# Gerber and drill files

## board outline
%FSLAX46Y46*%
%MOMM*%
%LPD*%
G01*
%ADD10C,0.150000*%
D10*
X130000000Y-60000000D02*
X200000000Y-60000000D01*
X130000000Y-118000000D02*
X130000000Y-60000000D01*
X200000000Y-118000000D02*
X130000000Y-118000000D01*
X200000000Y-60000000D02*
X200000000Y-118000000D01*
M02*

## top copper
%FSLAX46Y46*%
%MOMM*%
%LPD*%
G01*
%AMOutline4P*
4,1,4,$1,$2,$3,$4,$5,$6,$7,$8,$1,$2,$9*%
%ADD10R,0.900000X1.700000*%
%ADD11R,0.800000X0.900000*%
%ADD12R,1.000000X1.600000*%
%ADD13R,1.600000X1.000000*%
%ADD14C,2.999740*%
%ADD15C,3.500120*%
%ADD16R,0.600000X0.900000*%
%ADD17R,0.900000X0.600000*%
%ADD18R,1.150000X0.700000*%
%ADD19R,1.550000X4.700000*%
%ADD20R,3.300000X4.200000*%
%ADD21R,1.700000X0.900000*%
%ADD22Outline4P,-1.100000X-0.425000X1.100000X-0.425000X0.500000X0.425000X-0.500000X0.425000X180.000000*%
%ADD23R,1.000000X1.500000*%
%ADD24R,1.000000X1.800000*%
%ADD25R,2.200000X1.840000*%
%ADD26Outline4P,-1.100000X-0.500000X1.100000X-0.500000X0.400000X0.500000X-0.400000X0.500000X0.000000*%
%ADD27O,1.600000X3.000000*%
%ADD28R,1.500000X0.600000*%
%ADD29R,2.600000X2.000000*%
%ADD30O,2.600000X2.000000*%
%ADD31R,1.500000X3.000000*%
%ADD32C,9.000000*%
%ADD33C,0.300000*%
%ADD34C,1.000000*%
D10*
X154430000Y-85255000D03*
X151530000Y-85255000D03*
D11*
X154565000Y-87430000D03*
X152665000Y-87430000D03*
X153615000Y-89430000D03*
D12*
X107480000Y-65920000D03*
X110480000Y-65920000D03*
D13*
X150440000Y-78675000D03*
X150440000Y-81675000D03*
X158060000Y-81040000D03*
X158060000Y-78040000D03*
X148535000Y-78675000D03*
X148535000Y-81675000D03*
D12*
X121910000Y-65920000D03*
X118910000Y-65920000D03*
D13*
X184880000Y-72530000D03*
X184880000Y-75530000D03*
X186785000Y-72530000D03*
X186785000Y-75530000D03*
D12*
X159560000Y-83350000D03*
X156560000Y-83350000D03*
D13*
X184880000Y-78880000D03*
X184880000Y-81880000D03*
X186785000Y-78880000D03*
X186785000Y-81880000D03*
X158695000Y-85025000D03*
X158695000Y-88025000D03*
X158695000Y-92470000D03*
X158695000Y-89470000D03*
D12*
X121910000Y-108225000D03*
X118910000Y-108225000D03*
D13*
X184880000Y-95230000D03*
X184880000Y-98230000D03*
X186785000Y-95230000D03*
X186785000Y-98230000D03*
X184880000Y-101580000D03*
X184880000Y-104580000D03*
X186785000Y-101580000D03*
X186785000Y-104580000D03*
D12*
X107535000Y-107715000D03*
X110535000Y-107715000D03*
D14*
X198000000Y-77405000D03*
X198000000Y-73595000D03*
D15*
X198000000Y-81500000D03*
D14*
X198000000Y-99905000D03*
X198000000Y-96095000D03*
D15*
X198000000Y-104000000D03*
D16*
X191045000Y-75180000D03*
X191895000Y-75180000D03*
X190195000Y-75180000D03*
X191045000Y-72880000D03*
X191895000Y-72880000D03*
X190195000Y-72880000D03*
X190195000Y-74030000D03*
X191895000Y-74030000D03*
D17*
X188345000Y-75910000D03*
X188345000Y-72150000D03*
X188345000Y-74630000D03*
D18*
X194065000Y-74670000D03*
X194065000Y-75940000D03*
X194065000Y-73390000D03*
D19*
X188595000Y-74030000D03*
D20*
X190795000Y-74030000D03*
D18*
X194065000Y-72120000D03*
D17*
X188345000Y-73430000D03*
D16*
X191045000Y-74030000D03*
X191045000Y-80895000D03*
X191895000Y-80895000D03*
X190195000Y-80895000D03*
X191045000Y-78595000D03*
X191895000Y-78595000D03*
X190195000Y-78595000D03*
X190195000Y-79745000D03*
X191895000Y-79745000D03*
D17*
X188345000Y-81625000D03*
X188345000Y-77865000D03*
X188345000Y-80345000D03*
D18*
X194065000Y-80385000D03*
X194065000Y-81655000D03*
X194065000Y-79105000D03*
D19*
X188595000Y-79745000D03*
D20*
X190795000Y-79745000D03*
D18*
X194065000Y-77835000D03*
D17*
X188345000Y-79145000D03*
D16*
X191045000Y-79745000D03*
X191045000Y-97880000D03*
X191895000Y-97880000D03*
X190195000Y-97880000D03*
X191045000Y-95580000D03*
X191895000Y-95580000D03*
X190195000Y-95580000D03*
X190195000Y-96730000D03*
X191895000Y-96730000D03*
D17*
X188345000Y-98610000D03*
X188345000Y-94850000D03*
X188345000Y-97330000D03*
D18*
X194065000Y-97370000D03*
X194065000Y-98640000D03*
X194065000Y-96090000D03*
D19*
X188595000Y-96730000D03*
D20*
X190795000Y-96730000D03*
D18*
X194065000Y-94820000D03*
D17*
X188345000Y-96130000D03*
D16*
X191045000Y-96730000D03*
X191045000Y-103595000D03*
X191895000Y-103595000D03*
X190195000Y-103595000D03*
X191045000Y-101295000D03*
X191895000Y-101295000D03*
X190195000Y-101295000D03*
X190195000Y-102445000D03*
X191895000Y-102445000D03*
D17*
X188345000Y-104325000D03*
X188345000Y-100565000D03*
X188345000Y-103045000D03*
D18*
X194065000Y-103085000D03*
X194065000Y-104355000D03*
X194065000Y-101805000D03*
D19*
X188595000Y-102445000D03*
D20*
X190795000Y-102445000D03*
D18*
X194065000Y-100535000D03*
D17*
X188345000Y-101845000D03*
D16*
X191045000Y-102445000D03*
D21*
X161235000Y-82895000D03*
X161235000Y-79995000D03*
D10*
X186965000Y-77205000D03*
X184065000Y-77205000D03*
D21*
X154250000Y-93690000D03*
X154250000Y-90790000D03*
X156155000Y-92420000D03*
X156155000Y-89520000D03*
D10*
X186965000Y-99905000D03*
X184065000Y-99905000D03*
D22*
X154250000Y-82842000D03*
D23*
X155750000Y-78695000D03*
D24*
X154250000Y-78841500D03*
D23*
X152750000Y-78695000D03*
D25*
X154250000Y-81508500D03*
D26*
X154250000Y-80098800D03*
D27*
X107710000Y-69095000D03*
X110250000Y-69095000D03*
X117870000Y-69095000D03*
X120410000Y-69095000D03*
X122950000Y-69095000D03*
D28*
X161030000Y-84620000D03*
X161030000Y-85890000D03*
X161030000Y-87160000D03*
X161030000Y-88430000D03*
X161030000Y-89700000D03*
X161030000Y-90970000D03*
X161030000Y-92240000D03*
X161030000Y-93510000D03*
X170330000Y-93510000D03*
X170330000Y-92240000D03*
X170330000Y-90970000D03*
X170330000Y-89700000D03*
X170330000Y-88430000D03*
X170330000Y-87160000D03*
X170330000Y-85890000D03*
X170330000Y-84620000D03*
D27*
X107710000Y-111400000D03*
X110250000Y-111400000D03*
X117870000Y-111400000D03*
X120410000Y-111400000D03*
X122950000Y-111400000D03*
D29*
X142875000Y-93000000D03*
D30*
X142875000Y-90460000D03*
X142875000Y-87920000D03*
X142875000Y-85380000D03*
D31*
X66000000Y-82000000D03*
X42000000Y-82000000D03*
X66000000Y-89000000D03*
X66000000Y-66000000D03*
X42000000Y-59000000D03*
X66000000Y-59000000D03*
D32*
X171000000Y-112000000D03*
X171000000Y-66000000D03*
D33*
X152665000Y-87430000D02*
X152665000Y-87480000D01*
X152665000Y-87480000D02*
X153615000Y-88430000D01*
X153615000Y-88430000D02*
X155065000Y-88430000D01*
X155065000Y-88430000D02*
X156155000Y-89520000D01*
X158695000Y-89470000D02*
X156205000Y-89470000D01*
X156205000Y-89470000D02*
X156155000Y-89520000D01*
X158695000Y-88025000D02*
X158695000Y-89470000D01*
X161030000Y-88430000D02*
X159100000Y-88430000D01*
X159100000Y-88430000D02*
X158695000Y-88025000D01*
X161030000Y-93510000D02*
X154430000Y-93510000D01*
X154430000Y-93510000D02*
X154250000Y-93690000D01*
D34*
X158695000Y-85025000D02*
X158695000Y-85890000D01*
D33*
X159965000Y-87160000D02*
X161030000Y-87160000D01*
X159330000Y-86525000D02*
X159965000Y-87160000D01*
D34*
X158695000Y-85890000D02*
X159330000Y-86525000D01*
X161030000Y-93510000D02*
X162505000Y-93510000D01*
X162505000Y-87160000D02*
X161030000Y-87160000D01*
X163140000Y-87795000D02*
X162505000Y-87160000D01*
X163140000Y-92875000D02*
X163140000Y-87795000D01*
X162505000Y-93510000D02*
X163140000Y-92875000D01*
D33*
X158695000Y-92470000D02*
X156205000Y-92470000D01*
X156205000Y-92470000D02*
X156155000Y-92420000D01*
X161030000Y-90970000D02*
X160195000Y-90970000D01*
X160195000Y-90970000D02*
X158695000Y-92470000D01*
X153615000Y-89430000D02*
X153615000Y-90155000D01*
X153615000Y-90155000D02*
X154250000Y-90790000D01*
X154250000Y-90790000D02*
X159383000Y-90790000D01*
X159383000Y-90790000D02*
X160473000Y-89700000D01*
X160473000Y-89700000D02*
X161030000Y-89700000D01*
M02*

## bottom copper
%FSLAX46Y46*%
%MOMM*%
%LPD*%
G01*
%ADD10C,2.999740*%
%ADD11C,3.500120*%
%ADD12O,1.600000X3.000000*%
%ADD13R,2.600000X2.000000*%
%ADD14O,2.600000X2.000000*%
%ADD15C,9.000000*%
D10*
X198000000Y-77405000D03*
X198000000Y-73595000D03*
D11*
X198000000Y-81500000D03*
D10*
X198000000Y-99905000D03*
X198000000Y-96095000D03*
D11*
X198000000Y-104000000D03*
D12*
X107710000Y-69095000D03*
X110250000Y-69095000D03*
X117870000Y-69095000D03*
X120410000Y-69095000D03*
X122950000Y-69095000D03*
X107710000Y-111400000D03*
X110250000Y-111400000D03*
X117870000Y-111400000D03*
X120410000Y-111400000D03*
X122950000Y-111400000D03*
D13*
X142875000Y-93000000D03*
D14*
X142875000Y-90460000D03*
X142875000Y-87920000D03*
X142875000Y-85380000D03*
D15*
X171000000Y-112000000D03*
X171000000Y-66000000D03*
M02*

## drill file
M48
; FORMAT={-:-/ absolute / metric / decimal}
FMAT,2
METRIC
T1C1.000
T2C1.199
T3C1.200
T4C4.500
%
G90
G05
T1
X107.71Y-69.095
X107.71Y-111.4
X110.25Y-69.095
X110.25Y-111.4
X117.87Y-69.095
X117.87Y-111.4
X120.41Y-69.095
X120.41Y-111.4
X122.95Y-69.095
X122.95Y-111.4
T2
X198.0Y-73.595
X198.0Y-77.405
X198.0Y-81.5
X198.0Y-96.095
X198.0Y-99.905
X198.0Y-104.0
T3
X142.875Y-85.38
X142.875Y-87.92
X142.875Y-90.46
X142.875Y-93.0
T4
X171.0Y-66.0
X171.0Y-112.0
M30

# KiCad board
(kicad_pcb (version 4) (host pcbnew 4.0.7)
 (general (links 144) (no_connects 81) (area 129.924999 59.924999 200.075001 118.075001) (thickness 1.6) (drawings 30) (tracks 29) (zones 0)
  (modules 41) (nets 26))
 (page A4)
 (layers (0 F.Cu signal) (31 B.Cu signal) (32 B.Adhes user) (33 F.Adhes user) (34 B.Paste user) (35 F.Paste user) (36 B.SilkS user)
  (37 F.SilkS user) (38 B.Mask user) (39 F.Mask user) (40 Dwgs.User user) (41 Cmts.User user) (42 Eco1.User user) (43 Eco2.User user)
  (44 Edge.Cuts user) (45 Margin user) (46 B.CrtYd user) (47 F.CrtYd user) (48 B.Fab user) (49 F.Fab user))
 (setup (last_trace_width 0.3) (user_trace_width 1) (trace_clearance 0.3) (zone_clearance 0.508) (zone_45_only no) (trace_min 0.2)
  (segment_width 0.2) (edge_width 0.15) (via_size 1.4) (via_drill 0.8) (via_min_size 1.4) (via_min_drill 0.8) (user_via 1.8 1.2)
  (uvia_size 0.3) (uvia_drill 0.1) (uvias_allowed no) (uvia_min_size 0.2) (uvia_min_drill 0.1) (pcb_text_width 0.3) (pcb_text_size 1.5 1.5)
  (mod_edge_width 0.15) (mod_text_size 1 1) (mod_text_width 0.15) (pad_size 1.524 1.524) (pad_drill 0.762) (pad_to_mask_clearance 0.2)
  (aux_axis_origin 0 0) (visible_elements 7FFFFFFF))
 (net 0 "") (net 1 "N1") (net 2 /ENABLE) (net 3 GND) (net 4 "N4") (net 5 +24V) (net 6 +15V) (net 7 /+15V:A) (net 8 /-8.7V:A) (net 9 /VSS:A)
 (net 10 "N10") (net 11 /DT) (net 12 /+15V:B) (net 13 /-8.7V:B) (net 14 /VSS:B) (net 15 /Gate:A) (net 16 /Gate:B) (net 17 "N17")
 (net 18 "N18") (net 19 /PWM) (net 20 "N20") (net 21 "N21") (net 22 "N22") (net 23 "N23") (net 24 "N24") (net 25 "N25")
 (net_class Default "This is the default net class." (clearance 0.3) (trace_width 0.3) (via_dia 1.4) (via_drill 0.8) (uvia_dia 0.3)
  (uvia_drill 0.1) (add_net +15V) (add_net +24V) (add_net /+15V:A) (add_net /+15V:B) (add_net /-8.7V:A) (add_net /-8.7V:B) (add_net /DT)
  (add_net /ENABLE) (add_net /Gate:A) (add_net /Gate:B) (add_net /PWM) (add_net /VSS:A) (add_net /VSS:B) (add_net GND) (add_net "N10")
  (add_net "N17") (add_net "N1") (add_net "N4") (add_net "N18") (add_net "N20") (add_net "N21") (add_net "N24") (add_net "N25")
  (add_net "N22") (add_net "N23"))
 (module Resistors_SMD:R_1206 (layer F.Cu) (at 152.98 85.255 180)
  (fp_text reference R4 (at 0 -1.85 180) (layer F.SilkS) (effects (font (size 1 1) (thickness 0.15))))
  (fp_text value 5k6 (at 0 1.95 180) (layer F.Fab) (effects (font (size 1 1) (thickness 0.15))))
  (pad 1 smd rect (at -1.45 0 180) (size 0.9 1.7) (layers F.Cu F.Paste F.Mask) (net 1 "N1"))
  (pad 2 smd rect (at 1.45 0 180) (size 0.9 1.7) (layers F.Cu F.Paste F.Mask) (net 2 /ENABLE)))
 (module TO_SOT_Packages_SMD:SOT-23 (layer F.Cu) (at 153.615 88.43 270)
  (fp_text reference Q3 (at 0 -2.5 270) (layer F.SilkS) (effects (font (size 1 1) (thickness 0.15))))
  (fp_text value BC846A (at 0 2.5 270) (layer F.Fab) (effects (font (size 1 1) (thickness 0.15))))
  (pad 1 smd rect (at -1 -0.95 270) (size 0.9 0.8) (layers F.Cu F.Paste F.Mask) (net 1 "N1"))
  (pad 2 smd rect (at -1 0.95 270) (size 0.9 0.8) (layers F.Cu F.Paste F.Mask) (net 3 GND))
  (pad 3 smd rect (at 1 0 270) (size 0.9 0.8) (layers F.Cu F.Paste F.Mask) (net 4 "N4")))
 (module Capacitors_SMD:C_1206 (layer F.Cu) (at 108.98 65.92)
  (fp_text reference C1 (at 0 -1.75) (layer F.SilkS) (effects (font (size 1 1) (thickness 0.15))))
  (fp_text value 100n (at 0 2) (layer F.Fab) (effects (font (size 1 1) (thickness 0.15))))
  (pad 1 smd rect (at -1.5 0) (size 1 1.6) (layers F.Cu F.Paste F.Mask) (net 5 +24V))
  (pad 2 smd rect (at 1.5 0) (size 1 1.6) (layers F.Cu F.Paste F.Mask) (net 3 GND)))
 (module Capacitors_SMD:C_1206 (layer F.Cu) (at 150.44 80.175 270)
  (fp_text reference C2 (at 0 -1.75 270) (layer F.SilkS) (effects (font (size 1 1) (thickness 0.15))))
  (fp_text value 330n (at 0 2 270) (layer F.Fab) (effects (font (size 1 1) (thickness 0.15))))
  (pad 1 smd rect (at -1.5 0 270) (size 1 1.6) (layers F.Cu F.Paste F.Mask) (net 5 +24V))
  (pad 2 smd rect (at 1.5 0 270) (size 1 1.6) (layers F.Cu F.Paste F.Mask) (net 3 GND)))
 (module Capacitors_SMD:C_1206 (layer F.Cu) (at 158.06 79.54 90)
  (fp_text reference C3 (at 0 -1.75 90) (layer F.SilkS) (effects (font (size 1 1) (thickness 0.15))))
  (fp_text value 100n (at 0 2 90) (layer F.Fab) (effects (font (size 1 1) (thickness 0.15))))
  (pad 1 smd rect (at -1.5 0 90) (size 1 1.6) (layers F.Cu F.Paste F.Mask) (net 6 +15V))
  (pad 2 smd rect (at 1.5 0 90) (size 1 1.6) (layers F.Cu F.Paste F.Mask) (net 3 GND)))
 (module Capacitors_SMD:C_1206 (layer F.Cu) (at 148.535 80.175 270)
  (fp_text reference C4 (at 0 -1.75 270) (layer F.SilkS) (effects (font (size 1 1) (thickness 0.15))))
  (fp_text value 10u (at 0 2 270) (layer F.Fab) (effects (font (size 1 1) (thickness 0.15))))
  (pad 1 smd rect (at -1.5 0 270) (size 1 1.6) (layers F.Cu F.Paste F.Mask) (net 5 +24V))
  (pad 2 smd rect (at 1.5 0 270) (size 1 1.6) (layers F.Cu F.Paste F.Mask) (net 3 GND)))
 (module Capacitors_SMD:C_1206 (layer F.Cu) (at 120.41 65.92 180)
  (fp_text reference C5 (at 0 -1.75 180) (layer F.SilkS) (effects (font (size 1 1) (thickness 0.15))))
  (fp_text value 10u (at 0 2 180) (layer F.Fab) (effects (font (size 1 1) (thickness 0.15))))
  (pad 1 smd rect (at -1.5 0 180) (size 1 1.6) (layers F.Cu F.Paste F.Mask) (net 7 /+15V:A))
  (pad 2 smd rect (at 1.5 0 180) (size 1 1.6) (layers F.Cu F.Paste F.Mask) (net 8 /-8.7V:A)))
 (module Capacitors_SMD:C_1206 (layer F.Cu) (at 184.88 74.03 270)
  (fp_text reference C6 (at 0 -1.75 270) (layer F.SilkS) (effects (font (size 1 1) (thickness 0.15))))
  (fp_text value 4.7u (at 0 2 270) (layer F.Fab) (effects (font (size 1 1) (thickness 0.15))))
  (pad 1 smd rect (at -1.5 0 270) (size 1 1.6) (layers F.Cu F.Paste F.Mask) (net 7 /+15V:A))
  (pad 2 smd rect (at 1.5 0 270) (size 1 1.6) (layers F.Cu F.Paste F.Mask) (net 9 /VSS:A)))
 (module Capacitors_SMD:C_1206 (layer F.Cu) (at 186.785 74.03 270)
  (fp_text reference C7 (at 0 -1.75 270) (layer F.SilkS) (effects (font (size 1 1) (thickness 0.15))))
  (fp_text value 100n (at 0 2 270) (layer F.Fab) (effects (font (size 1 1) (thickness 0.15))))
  (pad 1 smd rect (at -1.5 0 270) (size 1 1.6) (layers F.Cu F.Paste F.Mask) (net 7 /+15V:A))
  (pad 2 smd rect (at 1.5 0 270) (size 1 1.6) (layers F.Cu F.Paste F.Mask) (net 9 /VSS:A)))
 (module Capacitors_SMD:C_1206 (layer F.Cu) (at 158.06 83.35 180)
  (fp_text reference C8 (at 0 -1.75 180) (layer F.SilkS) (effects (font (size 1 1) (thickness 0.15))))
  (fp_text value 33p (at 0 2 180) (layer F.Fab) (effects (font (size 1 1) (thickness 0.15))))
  (pad 1 smd rect (at -1.5 0 180) (size 1 1.6) (layers F.Cu F.Paste F.Mask) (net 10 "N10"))
  (pad 2 smd rect (at 1.5 0 180) (size 1 1.6) (layers F.Cu F.Paste F.Mask) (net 3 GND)))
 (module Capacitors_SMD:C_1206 (layer F.Cu) (at 184.88 80.38 270)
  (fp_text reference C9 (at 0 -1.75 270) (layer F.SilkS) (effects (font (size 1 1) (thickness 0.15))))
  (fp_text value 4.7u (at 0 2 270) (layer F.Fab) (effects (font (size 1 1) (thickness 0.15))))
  (pad 1 smd rect (at -1.5 0 270) (size 1 1.6) (layers F.Cu F.Paste F.Mask) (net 9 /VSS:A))
  (pad 2 smd rect (at 1.5 0 270) (size 1 1.6) (layers F.Cu F.Paste F.Mask) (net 8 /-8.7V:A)))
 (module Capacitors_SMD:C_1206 (layer F.Cu) (at 186.785 80.38 270)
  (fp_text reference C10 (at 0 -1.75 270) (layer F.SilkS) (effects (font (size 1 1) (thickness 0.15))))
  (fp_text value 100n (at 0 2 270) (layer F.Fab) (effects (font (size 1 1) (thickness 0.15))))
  (pad 1 smd rect (at -1.5 0 270) (size 1 1.6) (layers F.Cu F.Paste F.Mask) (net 9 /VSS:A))
  (pad 2 smd rect (at 1.5 0 270) (size 1 1.6) (layers F.Cu F.Paste F.Mask) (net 8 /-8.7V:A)))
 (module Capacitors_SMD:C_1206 (layer F.Cu) (at 158.695 86.525 270)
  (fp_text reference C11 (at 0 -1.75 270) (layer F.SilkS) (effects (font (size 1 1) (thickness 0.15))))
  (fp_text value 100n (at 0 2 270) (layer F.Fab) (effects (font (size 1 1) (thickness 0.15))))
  (pad 1 smd rect (at -1.5 0 270) (size 1 1.6) (layers F.Cu F.Paste F.Mask) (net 6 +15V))
  (pad 2 smd rect (at 1.5 0 270) (size 1 1.6) (layers F.Cu F.Paste F.Mask) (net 3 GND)))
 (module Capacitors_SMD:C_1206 (layer F.Cu) (at 158.695 90.97 90)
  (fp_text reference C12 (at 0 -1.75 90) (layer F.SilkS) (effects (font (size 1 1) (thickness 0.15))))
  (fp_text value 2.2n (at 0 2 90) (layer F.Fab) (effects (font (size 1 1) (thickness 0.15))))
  (pad 1 smd rect (at -1.5 0 90) (size 1 1.6) (layers F.Cu F.Paste F.Mask) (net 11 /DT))
  (pad 2 smd rect (at 1.5 0 90) (size 1 1.6) (layers F.Cu F.Paste F.Mask) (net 3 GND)))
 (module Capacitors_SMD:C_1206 (layer F.Cu) (at 120.41 108.225 180)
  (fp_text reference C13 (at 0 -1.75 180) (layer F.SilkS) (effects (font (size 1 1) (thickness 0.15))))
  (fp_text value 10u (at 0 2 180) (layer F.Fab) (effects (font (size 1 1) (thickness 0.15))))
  (pad 1 smd rect (at -1.5 0 180) (size 1 1.6) (layers F.Cu F.Paste F.Mask) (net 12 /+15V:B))
  (pad 2 smd rect (at 1.5 0 180) (size 1 1.6) (layers F.Cu F.Paste F.Mask) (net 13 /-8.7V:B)))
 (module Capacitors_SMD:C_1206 (layer F.Cu) (at 184.88 96.73 270)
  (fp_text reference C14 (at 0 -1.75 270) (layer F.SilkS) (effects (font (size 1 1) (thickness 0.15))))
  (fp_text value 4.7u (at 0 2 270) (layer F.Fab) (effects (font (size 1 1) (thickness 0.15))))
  (pad 1 smd rect (at -1.5 0 270) (size 1 1.6) (layers F.Cu F.Paste F.Mask) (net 12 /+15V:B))
  (pad 2 smd rect (at 1.5 0 270) (size 1 1.6) (layers F.Cu F.Paste F.Mask) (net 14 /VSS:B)))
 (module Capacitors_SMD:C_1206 (layer F.Cu) (at 186.785 96.73 270)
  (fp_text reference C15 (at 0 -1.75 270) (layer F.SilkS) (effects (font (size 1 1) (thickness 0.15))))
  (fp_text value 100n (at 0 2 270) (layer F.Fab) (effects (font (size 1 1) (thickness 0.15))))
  (pad 1 smd rect (at -1.5 0 270) (size 1 1.6) (layers F.Cu F.Paste F.Mask) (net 12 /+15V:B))
  (pad 2 smd rect (at 1.5 0 270) (size 1 1.6) (layers F.Cu F.Paste F.Mask) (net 14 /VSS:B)))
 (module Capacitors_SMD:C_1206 (layer F.Cu) (at 184.88 103.08 270)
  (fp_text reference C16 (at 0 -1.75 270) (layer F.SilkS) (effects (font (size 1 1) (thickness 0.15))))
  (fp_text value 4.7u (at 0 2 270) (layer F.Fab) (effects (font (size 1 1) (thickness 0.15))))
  (pad 1 smd rect (at -1.5 0 270) (size 1 1.6) (layers F.Cu F.Paste F.Mask) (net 14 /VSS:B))
  (pad 2 smd rect (at 1.5 0 270) (size 1 1.6) (layers F.Cu F.Paste F.Mask) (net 13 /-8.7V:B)))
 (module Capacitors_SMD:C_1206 (layer F.Cu) (at 186.785 103.08 270)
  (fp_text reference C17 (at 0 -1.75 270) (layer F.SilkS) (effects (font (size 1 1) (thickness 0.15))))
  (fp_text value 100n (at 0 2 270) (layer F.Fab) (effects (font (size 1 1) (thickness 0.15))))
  (pad 1 smd rect (at -1.5 0 270) (size 1 1.6) (layers F.Cu F.Paste F.Mask) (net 14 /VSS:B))
  (pad 2 smd rect (at 1.5 0 270) (size 1 1.6) (layers F.Cu F.Paste F.Mask) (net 13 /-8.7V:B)))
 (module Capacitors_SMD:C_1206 (layer F.Cu) (at 109.035 107.715)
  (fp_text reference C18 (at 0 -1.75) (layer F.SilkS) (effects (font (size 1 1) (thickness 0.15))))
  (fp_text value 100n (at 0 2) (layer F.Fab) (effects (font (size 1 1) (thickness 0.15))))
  (pad 1 smd rect (at -1.5 0) (size 1 1.6) (layers F.Cu F.Paste F.Mask) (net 5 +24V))
  (pad 2 smd rect (at 1.5 0) (size 1 1.6) (layers F.Cu F.Paste F.Mask) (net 3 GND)))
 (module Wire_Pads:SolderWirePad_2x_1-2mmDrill (layer F.Cu) (at 198 75.5 90)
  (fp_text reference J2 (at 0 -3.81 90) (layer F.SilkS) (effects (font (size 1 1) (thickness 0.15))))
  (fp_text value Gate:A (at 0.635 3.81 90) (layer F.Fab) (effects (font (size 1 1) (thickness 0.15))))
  (pad 1 thru_hole circle (at -1.905 0 90) (size 2.99974 2.99974) (drill 1.19888) (layers *.Cu *.Mask) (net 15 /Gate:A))
  (pad 1 thru_hole circle (at 1.905 0 90) (size 2.99974 2.99974) (drill 1.19888) (layers *.Cu *.Mask) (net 15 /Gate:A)))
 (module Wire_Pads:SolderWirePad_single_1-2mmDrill (layer F.Cu) (at 198 81.5)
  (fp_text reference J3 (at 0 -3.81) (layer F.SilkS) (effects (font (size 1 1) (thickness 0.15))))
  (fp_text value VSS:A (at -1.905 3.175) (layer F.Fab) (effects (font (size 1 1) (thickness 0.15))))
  (pad 1 thru_hole circle (at 0 0) (size 3.50012 3.50012) (drill 1.19888) (layers *.Cu *.Mask) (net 9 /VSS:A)))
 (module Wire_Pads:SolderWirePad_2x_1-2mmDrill (layer F.Cu) (at 198 98 90)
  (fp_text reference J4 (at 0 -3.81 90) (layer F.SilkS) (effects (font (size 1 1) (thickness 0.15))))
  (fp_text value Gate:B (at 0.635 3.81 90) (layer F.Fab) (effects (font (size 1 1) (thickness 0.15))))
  (pad 1 thru_hole circle (at -1.905 0 90) (size 2.99974 2.99974) (drill 1.19888) (layers *.Cu *.Mask) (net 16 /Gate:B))
  (pad 1 thru_hole circle (at 1.905 0 90) (size 2.99974 2.99974) (drill 1.19888) (layers *.Cu *.Mask) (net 16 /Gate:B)))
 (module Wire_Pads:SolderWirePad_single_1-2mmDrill (layer F.Cu) (at 198 104)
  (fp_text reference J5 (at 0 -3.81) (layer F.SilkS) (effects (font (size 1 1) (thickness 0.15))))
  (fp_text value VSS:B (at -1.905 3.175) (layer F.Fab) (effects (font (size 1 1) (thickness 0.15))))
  (pad 1 thru_hole circle (at 0 0) (size 3.50012 3.50012) (drill 1.19888) (layers *.Cu *.Mask) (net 14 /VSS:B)))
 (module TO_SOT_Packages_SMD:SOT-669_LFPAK (layer F.Cu) (at 191.23 74.03 180) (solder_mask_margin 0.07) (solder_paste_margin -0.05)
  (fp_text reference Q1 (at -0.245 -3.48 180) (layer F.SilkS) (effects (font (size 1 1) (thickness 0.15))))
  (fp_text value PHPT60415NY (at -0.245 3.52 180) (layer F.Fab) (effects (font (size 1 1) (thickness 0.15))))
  (pad 5 smd rect (at 0.185 -1.15 180) (size 0.6 0.9) (layers F.Cu F.Paste F.Mask) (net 7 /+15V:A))
  (pad 5 smd rect (at -0.665 -1.15 180) (size 0.6 0.9) (layers F.Cu F.Paste F.Mask) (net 7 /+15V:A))
  (pad 5 smd rect (at 1.035 -1.15 180) (size 0.6 0.9) (layers F.Cu F.Paste F.Mask) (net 7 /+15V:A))
  (pad 5 smd rect (at 0.185 1.15 180) (size 0.6 0.9) (layers F.Cu F.Paste F.Mask) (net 7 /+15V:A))
  (pad 5 smd rect (at -0.665 1.15 180) (size 0.6 0.9) (layers F.Cu F.Paste F.Mask) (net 7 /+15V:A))
  (pad 5 smd rect (at 1.035 1.15 180) (size 0.6 0.9) (layers F.Cu F.Paste F.Mask) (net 7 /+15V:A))
  (pad 5 smd rect (at 1.035 0 180) (size 0.6 0.9) (layers F.Cu F.Paste F.Mask) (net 7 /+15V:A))
  (pad 5 smd rect (at -0.665 0 180) (size 0.6 0.9) (layers F.Cu F.Paste F.Mask) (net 7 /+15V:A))
  (pad 5 smd rect (at 2.885 -1.88 90) (size 0.6 0.9) (layers F.Cu F.Paste F.Mask) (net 7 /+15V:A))
  (pad 5 smd rect (at 2.885 1.88 90) (size 0.6 0.9) (layers F.Cu F.Paste F.Mask) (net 7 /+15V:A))
  (pad 5 smd rect (at 2.885 -0.6 90) (size 0.6 0.9) (layers F.Cu F.Paste F.Mask) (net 7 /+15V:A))
  (pad 2 smd rect (at -2.835 -0.64 90) (size 0.7 1.15) (layers F.Cu F.Paste F.Mask) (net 15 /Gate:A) (solder_mask_margin 0.07)
   (solder_paste_margin -0.05))
  (pad 1 smd rect (at -2.835 -1.91 90) (size 0.7 1.15) (layers F.Cu F.Paste F.Mask) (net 15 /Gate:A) (solder_mask_margin 0.07)
   (solder_paste_margin -0.05))
  (pad 3 smd rect (at -2.835 0.64 90) (size 0.7 1.15) (layers F.Cu F.Paste F.Mask) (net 15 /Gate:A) (solder_mask_margin 0.07)
   (solder_paste_margin -0.05))
  (pad 5 smd rect (at 2.635 0 90) (size 4.7 1.55) (layers F.Cu F.Paste F.Mask) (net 7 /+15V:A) (solder_mask_margin 0.07))
  (pad 5 smd rect (at 0.435 0 90) (size 4.2 3.3) (layers F.Cu F.Paste F.Mask) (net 7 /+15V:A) (solder_mask_margin 0.07))
  (pad 4 smd rect (at -2.835 1.91 90) (size 0.7 1.15) (layers F.Cu F.Paste F.Mask) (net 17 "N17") (solder_mask_margin 0.07)
   (solder_paste_margin -0.05))
  (pad 5 smd rect (at 2.885 0.6 90) (size 0.6 0.9) (layers F.Cu F.Paste F.Mask) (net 7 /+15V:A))
  (pad 5 smd rect (at 0.185 0 180) (size 0.6 0.9) (layers F.Cu F.Paste F.Mask) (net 7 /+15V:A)))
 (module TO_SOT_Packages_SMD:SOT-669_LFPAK (layer F.Cu) (at 191.23 79.745 180) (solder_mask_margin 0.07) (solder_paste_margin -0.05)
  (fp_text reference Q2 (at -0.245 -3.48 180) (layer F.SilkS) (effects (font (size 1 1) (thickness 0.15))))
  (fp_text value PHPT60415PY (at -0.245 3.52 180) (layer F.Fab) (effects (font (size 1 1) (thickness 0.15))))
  (pad 5 smd rect (at 0.185 -1.15 180) (size 0.6 0.9) (layers F.Cu F.Paste F.Mask) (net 8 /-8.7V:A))
  (pad 5 smd rect (at -0.665 -1.15 180) (size 0.6 0.9) (layers F.Cu F.Paste F.Mask) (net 8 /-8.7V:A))
  (pad 5 smd rect (at 1.035 -1.15 180) (size 0.6 0.9) (layers F.Cu F.Paste F.Mask) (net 8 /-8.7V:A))
  (pad 5 smd rect (at 0.185 1.15 180) (size 0.6 0.9) (layers F.Cu F.Paste F.Mask) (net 8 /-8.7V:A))
  (pad 5 smd rect (at -0.665 1.15 180) (size 0.6 0.9) (layers F.Cu F.Paste F.Mask) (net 8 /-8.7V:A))
  (pad 5 smd rect (at 1.035 1.15 180) (size 0.6 0.9) (layers F.Cu F.Paste F.Mask) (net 8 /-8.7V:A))
  (pad 5 smd rect (at 1.035 0 180) (size 0.6 0.9) (layers F.Cu F.Paste F.Mask) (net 8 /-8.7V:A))
  (pad 5 smd rect (at -0.665 0 180) (size 0.6 0.9) (layers F.Cu F.Paste F.Mask) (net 8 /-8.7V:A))
  (pad 5 smd rect (at 2.885 -1.88 90) (size 0.6 0.9) (layers F.Cu F.Paste F.Mask) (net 8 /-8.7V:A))
  (pad 5 smd rect (at 2.885 1.88 90) (size 0.6 0.9) (layers F.Cu F.Paste F.Mask) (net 8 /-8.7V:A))
  (pad 5 smd rect (at 2.885 -0.6 90) (size 0.6 0.9) (layers F.Cu F.Paste F.Mask) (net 8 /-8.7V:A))
  (pad 2 smd rect (at -2.835 -0.64 90) (size 0.7 1.15) (layers F.Cu F.Paste F.Mask) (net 15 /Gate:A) (solder_mask_margin 0.07)
   (solder_paste_margin -0.05))
  (pad 1 smd rect (at -2.835 -1.91 90) (size 0.7 1.15) (layers F.Cu F.Paste F.Mask) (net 15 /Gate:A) (solder_mask_margin 0.07)
   (solder_paste_margin -0.05))
  (pad 3 smd rect (at -2.835 0.64 90) (size 0.7 1.15) (layers F.Cu F.Paste F.Mask) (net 15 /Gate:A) (solder_mask_margin 0.07)
   (solder_paste_margin -0.05))
  (pad 5 smd rect (at 2.635 0 90) (size 4.7 1.55) (layers F.Cu F.Paste F.Mask) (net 8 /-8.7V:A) (solder_mask_margin 0.07))
  (pad 5 smd rect (at 0.435 0 90) (size 4.2 3.3) (layers F.Cu F.Paste F.Mask) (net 8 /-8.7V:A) (solder_mask_margin 0.07))
  (pad 4 smd rect (at -2.835 1.91 90) (size 0.7 1.15) (layers F.Cu F.Paste F.Mask) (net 17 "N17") (solder_mask_margin 0.07)
   (solder_paste_margin -0.05))
  (pad 5 smd rect (at 2.885 0.6 90) (size 0.6 0.9) (layers F.Cu F.Paste F.Mask) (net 8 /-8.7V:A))
  (pad 5 smd rect (at 0.185 0 180) (size 0.6 0.9) (layers F.Cu F.Paste F.Mask) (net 8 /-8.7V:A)))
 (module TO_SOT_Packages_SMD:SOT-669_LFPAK (layer F.Cu) (at 191.23 96.73 180) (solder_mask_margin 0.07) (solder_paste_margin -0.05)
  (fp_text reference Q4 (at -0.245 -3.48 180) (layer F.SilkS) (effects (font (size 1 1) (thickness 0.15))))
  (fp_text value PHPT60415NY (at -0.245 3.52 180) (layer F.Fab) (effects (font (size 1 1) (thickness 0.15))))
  (pad 5 smd rect (at 0.185 -1.15 180) (size 0.6 0.9) (layers F.Cu F.Paste F.Mask) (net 12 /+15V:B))
  (pad 5 smd rect (at -0.665 -1.15 180) (size 0.6 0.9) (layers F.Cu F.Paste F.Mask) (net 12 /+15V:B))
  (pad 5 smd rect (at 1.035 -1.15 180) (size 0.6 0.9) (layers F.Cu F.Paste F.Mask) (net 12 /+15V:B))
  (pad 5 smd rect (at 0.185 1.15 180) (size 0.6 0.9) (layers F.Cu F.Paste F.Mask) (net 12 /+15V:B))
  (pad 5 smd rect (at -0.665 1.15 180) (size 0.6 0.9) (layers F.Cu F.Paste F.Mask) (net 12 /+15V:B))
  (pad 5 smd rect (at 1.035 1.15 180) (size 0.6 0.9) (layers F.Cu F.Paste F.Mask) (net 12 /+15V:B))
  (pad 5 smd rect (at 1.035 0 180) (size 0.6 0.9) (layers F.Cu F.Paste F.Mask) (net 12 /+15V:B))
  (pad 5 smd rect (at -0.665 0 180) (size 0.6 0.9) (layers F.Cu F.Paste F.Mask) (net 12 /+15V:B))
  (pad 5 smd rect (at 2.885 -1.88 90) (size 0.6 0.9) (layers F.Cu F.Paste F.Mask) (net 12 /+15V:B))
  (pad 5 smd rect (at 2.885 1.88 90) (size 0.6 0.9) (layers F.Cu F.Paste F.Mask) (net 12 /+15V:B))
  (pad 5 smd rect (at 2.885 -0.6 90) (size 0.6 0.9) (layers F.Cu F.Paste F.Mask) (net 12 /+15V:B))
  (pad 2 smd rect (at -2.835 -0.64 90) (size 0.7 1.15) (layers F.Cu F.Paste F.Mask) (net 16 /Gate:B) (solder_mask_margin 0.07)
   (solder_paste_margin -0.05))
  (pad 1 smd rect (at -2.835 -1.91 90) (size 0.7 1.15) (layers F.Cu F.Paste F.Mask) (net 16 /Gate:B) (solder_mask_margin 0.07)
   (solder_paste_margin -0.05))
  (pad 3 smd rect (at -2.835 0.64 90) (size 0.7 1.15) (layers F.Cu F.Paste F.Mask) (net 16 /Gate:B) (solder_mask_margin 0.07)
   (solder_paste_margin -0.05))
  (pad 5 smd rect (at 2.635 0 90) (size 4.7 1.55) (layers F.Cu F.Paste F.Mask) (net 12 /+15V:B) (solder_mask_margin 0.07))
  (pad 5 smd rect (at 0.435 0 90) (size 4.2 3.3) (layers F.Cu F.Paste F.Mask) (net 12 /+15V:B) (solder_mask_margin 0.07))
  (pad 4 smd rect (at -2.835 1.91 90) (size 0.7 1.15) (layers F.Cu F.Paste F.Mask) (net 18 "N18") (solder_mask_margin 0.07)
   (solder_paste_margin -0.05))
  (pad 5 smd rect (at 2.885 0.6 90) (size 0.6 0.9) (layers F.Cu F.Paste F.Mask) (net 12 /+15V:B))
  (pad 5 smd rect (at 0.185 0 180) (size 0.6 0.9) (layers F.Cu F.Paste F.Mask) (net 12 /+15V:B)))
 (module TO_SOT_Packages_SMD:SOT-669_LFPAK (layer F.Cu) (at 191.23 102.445 180) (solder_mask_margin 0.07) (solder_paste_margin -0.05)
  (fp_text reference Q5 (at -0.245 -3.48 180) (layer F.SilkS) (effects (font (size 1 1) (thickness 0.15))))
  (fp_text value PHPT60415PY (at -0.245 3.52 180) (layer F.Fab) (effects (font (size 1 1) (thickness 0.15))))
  (pad 5 smd rect (at 0.185 -1.15 180) (size 0.6 0.9) (layers F.Cu F.Paste F.Mask) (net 13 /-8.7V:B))
  (pad 5 smd rect (at -0.665 -1.15 180) (size 0.6 0.9) (layers F.Cu F.Paste F.Mask) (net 13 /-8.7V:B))
  (pad 5 smd rect (at 1.035 -1.15 180) (size 0.6 0.9) (layers F.Cu F.Paste F.Mask) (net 13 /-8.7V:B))
  (pad 5 smd rect (at 0.185 1.15 180) (size 0.6 0.9) (layers F.Cu F.Paste F.Mask) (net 13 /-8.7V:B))
  (pad 5 smd rect (at -0.665 1.15 180) (size 0.6 0.9) (layers F.Cu F.Paste F.Mask) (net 13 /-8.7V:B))
  (pad 5 smd rect (at 1.035 1.15 180) (size 0.6 0.9) (layers F.Cu F.Paste F.Mask) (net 13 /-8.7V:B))
  (pad 5 smd rect (at 1.035 0 180) (size 0.6 0.9) (layers F.Cu F.Paste F.Mask) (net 13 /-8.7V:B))
  (pad 5 smd rect (at -0.665 0 180) (size 0.6 0.9) (layers F.Cu F.Paste F.Mask) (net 13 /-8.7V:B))
  (pad 5 smd rect (at 2.885 -1.88 90) (size 0.6 0.9) (layers F.Cu F.Paste F.Mask) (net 13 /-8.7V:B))
  (pad 5 smd rect (at 2.885 1.88 90) (size 0.6 0.9) (layers F.Cu F.Paste F.Mask) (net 13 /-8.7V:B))
  (pad 5 smd rect (at 2.885 -0.6 90) (size 0.6 0.9) (layers F.Cu F.Paste F.Mask) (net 13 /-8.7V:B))
  (pad 2 smd rect (at -2.835 -0.64 90) (size 0.7 1.15) (layers F.Cu F.Paste F.Mask) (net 16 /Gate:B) (solder_mask_margin 0.07)
   (solder_paste_margin -0.05))
  (pad 1 smd rect (at -2.835 -1.91 90) (size 0.7 1.15) (layers F.Cu F.Paste F.Mask) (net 16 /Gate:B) (solder_mask_margin 0.07)
   (solder_paste_margin -0.05))
  (pad 3 smd rect (at -2.835 0.64 90) (size 0.7 1.15) (layers F.Cu F.Paste F.Mask) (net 16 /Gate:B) (solder_mask_margin 0.07)
   (solder_paste_margin -0.05))
  (pad 5 smd rect (at 2.635 0 90) (size 4.7 1.55) (layers F.Cu F.Paste F.Mask) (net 13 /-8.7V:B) (solder_mask_margin 0.07))
  (pad 5 smd rect (at 0.435 0 90) (size 4.2 3.3) (layers F.Cu F.Paste F.Mask) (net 13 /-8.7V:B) (solder_mask_margin 0.07))
  (pad 4 smd rect (at -2.835 1.91 90) (size 0.7 1.15) (layers F.Cu F.Paste F.Mask) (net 18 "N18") (solder_mask_margin 0.07)
   (solder_paste_margin -0.05))
  (pad 5 smd rect (at 2.885 0.6 90) (size 0.6 0.9) (layers F.Cu F.Paste F.Mask) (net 13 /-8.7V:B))
  (pad 5 smd rect (at 0.185 0 180) (size 0.6 0.9) (layers F.Cu F.Paste F.Mask) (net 13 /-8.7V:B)))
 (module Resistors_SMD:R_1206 (layer F.Cu) (at 161.235 81.445 90)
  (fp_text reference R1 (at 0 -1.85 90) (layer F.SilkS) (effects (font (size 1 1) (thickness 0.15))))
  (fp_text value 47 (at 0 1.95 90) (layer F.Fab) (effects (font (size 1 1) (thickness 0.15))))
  (pad 1 smd rect (at -1.45 0 90) (size 0.9 1.7) (layers F.Cu F.Paste F.Mask) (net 10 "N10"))
  (pad 2 smd rect (at 1.45 0 90) (size 0.9 1.7) (layers F.Cu F.Paste F.Mask) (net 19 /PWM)))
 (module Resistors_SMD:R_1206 (layer F.Cu) (at 185.515 77.205 180)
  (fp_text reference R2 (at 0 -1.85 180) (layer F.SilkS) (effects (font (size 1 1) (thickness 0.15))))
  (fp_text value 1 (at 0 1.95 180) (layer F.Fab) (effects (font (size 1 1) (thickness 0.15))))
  (pad 1 smd rect (at -1.45 0 180) (size 0.9 1.7) (layers F.Cu F.Paste F.Mask) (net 17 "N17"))
  (pad 2 smd rect (at 1.45 0 180) (size 0.9 1.7) (layers F.Cu F.Paste F.Mask) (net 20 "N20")))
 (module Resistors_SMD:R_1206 (layer F.Cu) (at 154.25 92.24 90)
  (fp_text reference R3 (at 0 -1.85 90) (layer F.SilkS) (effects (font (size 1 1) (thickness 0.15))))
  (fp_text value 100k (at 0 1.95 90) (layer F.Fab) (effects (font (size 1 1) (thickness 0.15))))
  (pad 1 smd rect (at -1.45 0 90) (size 0.9 1.7) (layers F.Cu F.Paste F.Mask) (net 6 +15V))
  (pad 2 smd rect (at 1.45 0 90) (size 0.9 1.7) (layers F.Cu F.Paste F.Mask) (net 4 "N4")))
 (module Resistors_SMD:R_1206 (layer F.Cu) (at 156.155 90.97 90)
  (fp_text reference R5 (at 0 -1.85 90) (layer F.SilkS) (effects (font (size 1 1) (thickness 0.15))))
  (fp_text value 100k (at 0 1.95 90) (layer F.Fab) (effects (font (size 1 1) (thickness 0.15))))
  (pad 1 smd rect (at -1.45 0 90) (size 0.9 1.7) (layers F.Cu F.Paste F.Mask) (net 11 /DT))
  (pad 2 smd rect (at 1.45 0 90) (size 0.9 1.7) (layers F.Cu F.Paste F.Mask) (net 3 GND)))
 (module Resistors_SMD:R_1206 (layer F.Cu) (at 185.515 99.905 180)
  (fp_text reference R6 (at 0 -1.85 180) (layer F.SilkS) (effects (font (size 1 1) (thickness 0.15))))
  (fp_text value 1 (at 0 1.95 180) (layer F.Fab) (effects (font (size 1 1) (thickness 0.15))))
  (pad 1 smd rect (at -1.45 0 180) (size 0.9 1.7) (layers F.Cu F.Paste F.Mask) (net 18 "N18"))
  (pad 2 smd rect (at 1.45 0 180) (size 0.9 1.7) (layers F.Cu F.Paste F.Mask) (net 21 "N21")))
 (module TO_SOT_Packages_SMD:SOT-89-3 (layer F.Cu) (at 154.25 80.175 270)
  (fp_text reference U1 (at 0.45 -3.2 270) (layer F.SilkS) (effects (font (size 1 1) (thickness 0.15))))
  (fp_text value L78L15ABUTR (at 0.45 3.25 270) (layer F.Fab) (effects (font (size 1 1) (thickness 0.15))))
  (pad 2 smd trapezoid (at 2.667 0 180) (size 1.6 0.85) (rect_delta 0 0.6) (layers F.Cu F.Paste F.Mask) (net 3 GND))
  (pad 1 smd rect (at -1.48 -1.5 180) (size 1 1.5) (layers F.Cu F.Paste F.Mask) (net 6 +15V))
  (pad 2 smd rect (at -1.3335 0 180) (size 1 1.8) (layers F.Cu F.Paste F.Mask) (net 3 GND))
  (pad 3 smd rect (at -1.48 1.5 180) (size 1 1.5) (layers F.Cu F.Paste F.Mask) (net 5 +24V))
  (pad 2 smd rect (at 1.3335 0 180) (size 2.2 1.84) (layers F.Cu F.Paste F.Mask) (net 3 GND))
  (pad 2 smd trapezoid (at -0.0762 0) (size 1.5 1) (rect_delta 0 0.7) (layers F.Cu F.Paste F.Mask) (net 3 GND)))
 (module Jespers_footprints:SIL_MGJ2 (layer B.Cu) (at 107.71 69.095)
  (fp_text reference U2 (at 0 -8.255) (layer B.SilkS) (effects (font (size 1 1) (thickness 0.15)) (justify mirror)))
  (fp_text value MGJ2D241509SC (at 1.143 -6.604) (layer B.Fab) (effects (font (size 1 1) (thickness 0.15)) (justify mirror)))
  (pad 1 thru_hole oval (at 0 0) (size 1.6 3) (drill 1) (layers *.Cu *.Mask) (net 5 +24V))
  (pad 2 thru_hole oval (at 2.54 0) (size 1.6 3) (drill 1) (layers *.Cu *.Mask) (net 3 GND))
  (pad 5 thru_hole oval (at 10.16 0) (size 1.6 3) (drill 1) (layers *.Cu *.Mask) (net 8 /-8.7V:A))
  (pad 6 thru_hole oval (at 12.7 0) (size 1.6 3) (drill 1) (layers *.Cu *.Mask) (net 9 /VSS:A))
  (pad 7 thru_hole oval (at 15.24 0) (size 1.6 3) (drill 1) (layers *.Cu *.Mask) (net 7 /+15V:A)))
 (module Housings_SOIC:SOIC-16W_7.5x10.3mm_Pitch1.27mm (layer F.Cu) (at 165.68 89.065)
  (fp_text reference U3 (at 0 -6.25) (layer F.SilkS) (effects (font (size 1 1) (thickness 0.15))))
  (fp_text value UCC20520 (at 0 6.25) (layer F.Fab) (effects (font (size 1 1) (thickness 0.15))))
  (pad 1 smd rect (at -4.65 -4.445) (size 1.5 0.6) (layers F.Cu F.Paste F.Mask) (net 10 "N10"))
  (pad 2 smd rect (at -4.65 -3.175) (size 1.5 0.6) (layers F.Cu F.Paste F.Mask) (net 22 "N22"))
  (pad 3 smd rect (at -4.65 -1.905) (size 1.5 0.6) (layers F.Cu F.Paste F.Mask) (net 6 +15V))
  (pad 4 smd rect (at -4.65 -0.635) (size 1.5 0.6) (layers F.Cu F.Paste F.Mask) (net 3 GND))
  (pad 5 smd rect (at -4.65 0.635) (size 1.5 0.6) (layers F.Cu F.Paste F.Mask) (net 4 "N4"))
  (pad 6 smd rect (at -4.65 1.905) (size 1.5 0.6) (layers F.Cu F.Paste F.Mask) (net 11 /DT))
  (pad 7 smd rect (at -4.65 3.175) (size 1.5 0.6) (layers F.Cu F.Paste F.Mask) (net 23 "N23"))
  (pad 8 smd rect (at -4.65 4.445) (size 1.5 0.6) (layers F.Cu F.Paste F.Mask) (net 6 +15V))
  (pad 9 smd rect (at 4.65 4.445) (size 1.5 0.6) (layers F.Cu F.Paste F.Mask) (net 13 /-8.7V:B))
  (pad 10 smd rect (at 4.65 3.175) (size 1.5 0.6) (layers F.Cu F.Paste F.Mask) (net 21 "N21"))
  (pad 11 smd rect (at 4.65 1.905) (size 1.5 0.6) (layers F.Cu F.Paste F.Mask) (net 12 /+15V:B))
  (pad 12 smd rect (at 4.65 0.635) (size 1.5 0.6) (layers F.Cu F.Paste F.Mask) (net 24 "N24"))
  (pad 13 smd rect (at 4.65 -0.635) (size 1.5 0.6) (layers F.Cu F.Paste F.Mask) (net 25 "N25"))
  (pad 14 smd rect (at 4.65 -1.905) (size 1.5 0.6) (layers F.Cu F.Paste F.Mask) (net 8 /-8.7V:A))
  (pad 15 smd rect (at 4.65 -3.175) (size 1.5 0.6) (layers F.Cu F.Paste F.Mask) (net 20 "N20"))
  (pad 16 smd rect (at 4.65 -4.445) (size 1.5 0.6) (layers F.Cu F.Paste F.Mask) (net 7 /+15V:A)))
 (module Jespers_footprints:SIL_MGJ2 (layer B.Cu) (at 107.71 111.4)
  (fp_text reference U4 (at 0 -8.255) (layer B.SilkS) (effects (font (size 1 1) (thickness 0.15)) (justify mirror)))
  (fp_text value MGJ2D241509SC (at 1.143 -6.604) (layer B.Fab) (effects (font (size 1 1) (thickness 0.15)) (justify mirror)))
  (pad 1 thru_hole oval (at 0 0) (size 1.6 3) (drill 1) (layers *.Cu *.Mask) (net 5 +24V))
  (pad 2 thru_hole oval (at 2.54 0) (size 1.6 3) (drill 1) (layers *.Cu *.Mask) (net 3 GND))
  (pad 5 thru_hole oval (at 10.16 0) (size 1.6 3) (drill 1) (layers *.Cu *.Mask) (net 13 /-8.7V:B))
  (pad 6 thru_hole oval (at 12.7 0) (size 1.6 3) (drill 1) (layers *.Cu *.Mask) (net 14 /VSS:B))
  (pad 7 thru_hole oval (at 15.24 0) (size 1.6 3) (drill 1) (layers *.Cu *.Mask) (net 12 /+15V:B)))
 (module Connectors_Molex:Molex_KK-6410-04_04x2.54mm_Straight (layer B.Cu) (at 142.875 93 90)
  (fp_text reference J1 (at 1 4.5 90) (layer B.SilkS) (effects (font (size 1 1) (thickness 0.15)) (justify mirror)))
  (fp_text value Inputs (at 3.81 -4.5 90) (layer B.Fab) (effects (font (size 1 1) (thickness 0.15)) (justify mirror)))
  (pad 1 thru_hole rect (at 0 0 90) (size 2 2.6) (drill 1.2) (layers *.Cu *.Mask) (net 19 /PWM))
  (pad 2 thru_hole oval (at 2.54 0 90) (size 2 2.6) (drill 1.2) (layers *.Cu *.Mask) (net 2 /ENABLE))
  (pad 3 thru_hole oval (at 5.08 0 90) (size 2 2.6) (drill 1.2) (layers *.Cu *.Mask) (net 5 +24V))
  (pad 4 thru_hole oval (at 7.62 0 90) (size 2 2.6) (drill 1.2) (layers *.Cu *.Mask) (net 3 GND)))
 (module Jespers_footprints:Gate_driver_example (layer F.Cu) (at 66 59 270)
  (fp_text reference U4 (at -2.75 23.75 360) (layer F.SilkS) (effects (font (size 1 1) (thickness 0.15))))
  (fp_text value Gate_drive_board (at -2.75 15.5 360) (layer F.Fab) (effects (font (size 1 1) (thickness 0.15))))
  (pad 5 smd rect (at 23 0 270) (size 3 1.5) (layers F.Cu F.Paste F.Mask))
  (pad 4 smd rect (at 23 24 270) (size 3 1.5) (layers F.Cu F.Paste F.Mask))
  (pad 6 smd rect (at 30 0 270) (size 3 1.5) (layers F.Cu F.Paste F.Mask))
  (pad 3 smd rect (at 7 0 270) (size 3 1.5) (layers F.Cu F.Paste F.Mask))
  (pad 1 smd rect (at 0 24 270) (size 3 1.5) (layers F.Cu F.Paste F.Mask))
  (pad 2 smd rect (at 0 0 270) (size 3 1.5) (layers F.Cu F.Paste F.Mask)))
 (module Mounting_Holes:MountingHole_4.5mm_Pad (layer F.Cu) (at 171 112)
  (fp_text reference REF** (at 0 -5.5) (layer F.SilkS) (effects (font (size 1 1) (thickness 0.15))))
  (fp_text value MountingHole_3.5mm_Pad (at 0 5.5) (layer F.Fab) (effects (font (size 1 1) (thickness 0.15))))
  (pad 1 thru_hole circle (at 0 0) (size 9 9) (drill 4.5) (layers *.Cu *.Mask)))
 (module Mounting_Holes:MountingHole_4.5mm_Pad (layer F.Cu) (at 171 66)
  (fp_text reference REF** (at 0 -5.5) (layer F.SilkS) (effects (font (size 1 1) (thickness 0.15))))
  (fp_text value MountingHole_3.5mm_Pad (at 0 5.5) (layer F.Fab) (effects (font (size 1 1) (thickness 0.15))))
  (pad 1 thru_hole circle (at 0 0) (size 9 9) (drill 4.5) (layers *.Cu *.Mask)))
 (gr_line (start 130 60) (end 200 60) (angle 90) (layer Edge.Cuts) (width 0.15))
 (gr_line (start 130 118) (end 130 60) (angle 90) (layer Edge.Cuts) (width 0.15))
 (gr_line (start 200 118) (end 130 118) (angle 90) (layer Edge.Cuts) (width 0.15))
 (gr_line (start 200 60) (end 200 118) (angle 90) (layer Edge.Cuts) (width 0.15))
 (segment (start 152.665 87.43) (end 152.665 87.48) (width 0.3) (layer F.Cu) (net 3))
 (segment (start 152.665 87.48) (end 153.615 88.43) (width 0.3) (layer F.Cu) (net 3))
 (segment (start 153.615 88.43) (end 155.065 88.43) (width 0.3) (layer F.Cu) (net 3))
 (segment (start 155.065 88.43) (end 156.155 89.52) (width 0.3) (layer F.Cu) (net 3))
 (segment (start 158.695 89.47) (end 156.205 89.47) (width 0.3) (layer F.Cu) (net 3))
 (segment (start 156.205 89.47) (end 156.155 89.52) (width 0.3) (layer F.Cu) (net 3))
 (segment (start 158.695 88.025) (end 158.695 89.47) (width 0.3) (layer F.Cu) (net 3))
 (segment (start 161.03 88.43) (end 159.1 88.43) (width 0.3) (layer F.Cu) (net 3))
 (segment (start 159.1 88.43) (end 158.695 88.025) (width 0.3) (layer F.Cu) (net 3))
 (segment (start 161.03 93.51) (end 154.43 93.51) (width 0.3) (layer F.Cu) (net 6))
 (segment (start 154.43 93.51) (end 154.25 93.69) (width 0.3) (layer F.Cu) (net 6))
 (segment (start 158.695 85.025) (end 158.695 85.89) (width 1) (layer F.Cu) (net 6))
 (segment (start 159.965 87.16) (end 161.03 87.16) (width 0.3) (layer F.Cu) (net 6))
 (segment (start 159.33 86.525) (end 159.965 87.16) (width 0.3) (layer F.Cu) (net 6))
 (segment (start 158.695 85.89) (end 159.33 86.525) (width 1) (layer F.Cu) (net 6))
 (segment (start 161.03 93.51) (end 162.505 93.51) (width 1) (layer F.Cu) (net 6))
 (segment (start 162.505 87.16) (end 161.03 87.16) (width 1) (layer F.Cu) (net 6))
 (segment (start 163.14 87.795) (end 162.505 87.16) (width 1) (layer F.Cu) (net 6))
 (segment (start 163.14 92.875) (end 163.14 87.795) (width 1) (layer F.Cu) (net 6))
 (segment (start 162.505 93.51) (end 163.14 92.875) (width 1) (layer F.Cu) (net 6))
 (segment (start 158.695 92.47) (end 156.205 92.47) (width 0.3) (layer F.Cu) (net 11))
 (segment (start 156.205 92.47) (end 156.155 92.42) (width 0.3) (layer F.Cu) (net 11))
 (segment (start 161.03 90.97) (end 160.195 90.97) (width 0.3) (layer F.Cu) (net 11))
 (segment (start 160.195 90.97) (end 158.695 92.47) (width 0.3) (layer F.Cu) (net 11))
 (segment (start 153.615 89.43) (end 153.615 90.155) (width 0.3) (layer F.Cu) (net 4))
 (segment (start 153.615 90.155) (end 154.25 90.79) (width 0.3) (layer F.Cu) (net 4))
 (segment (start 154.25 90.79) (end 159.383 90.79) (width 0.3) (layer F.Cu) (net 4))
 (segment (start 159.383 90.79) (end 160.473 89.7) (width 0.3) (layer F.Cu) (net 4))
 (segment (start 160.473 89.7) (end 161.03 89.7) (width 0.3) (layer F.Cu) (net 4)))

